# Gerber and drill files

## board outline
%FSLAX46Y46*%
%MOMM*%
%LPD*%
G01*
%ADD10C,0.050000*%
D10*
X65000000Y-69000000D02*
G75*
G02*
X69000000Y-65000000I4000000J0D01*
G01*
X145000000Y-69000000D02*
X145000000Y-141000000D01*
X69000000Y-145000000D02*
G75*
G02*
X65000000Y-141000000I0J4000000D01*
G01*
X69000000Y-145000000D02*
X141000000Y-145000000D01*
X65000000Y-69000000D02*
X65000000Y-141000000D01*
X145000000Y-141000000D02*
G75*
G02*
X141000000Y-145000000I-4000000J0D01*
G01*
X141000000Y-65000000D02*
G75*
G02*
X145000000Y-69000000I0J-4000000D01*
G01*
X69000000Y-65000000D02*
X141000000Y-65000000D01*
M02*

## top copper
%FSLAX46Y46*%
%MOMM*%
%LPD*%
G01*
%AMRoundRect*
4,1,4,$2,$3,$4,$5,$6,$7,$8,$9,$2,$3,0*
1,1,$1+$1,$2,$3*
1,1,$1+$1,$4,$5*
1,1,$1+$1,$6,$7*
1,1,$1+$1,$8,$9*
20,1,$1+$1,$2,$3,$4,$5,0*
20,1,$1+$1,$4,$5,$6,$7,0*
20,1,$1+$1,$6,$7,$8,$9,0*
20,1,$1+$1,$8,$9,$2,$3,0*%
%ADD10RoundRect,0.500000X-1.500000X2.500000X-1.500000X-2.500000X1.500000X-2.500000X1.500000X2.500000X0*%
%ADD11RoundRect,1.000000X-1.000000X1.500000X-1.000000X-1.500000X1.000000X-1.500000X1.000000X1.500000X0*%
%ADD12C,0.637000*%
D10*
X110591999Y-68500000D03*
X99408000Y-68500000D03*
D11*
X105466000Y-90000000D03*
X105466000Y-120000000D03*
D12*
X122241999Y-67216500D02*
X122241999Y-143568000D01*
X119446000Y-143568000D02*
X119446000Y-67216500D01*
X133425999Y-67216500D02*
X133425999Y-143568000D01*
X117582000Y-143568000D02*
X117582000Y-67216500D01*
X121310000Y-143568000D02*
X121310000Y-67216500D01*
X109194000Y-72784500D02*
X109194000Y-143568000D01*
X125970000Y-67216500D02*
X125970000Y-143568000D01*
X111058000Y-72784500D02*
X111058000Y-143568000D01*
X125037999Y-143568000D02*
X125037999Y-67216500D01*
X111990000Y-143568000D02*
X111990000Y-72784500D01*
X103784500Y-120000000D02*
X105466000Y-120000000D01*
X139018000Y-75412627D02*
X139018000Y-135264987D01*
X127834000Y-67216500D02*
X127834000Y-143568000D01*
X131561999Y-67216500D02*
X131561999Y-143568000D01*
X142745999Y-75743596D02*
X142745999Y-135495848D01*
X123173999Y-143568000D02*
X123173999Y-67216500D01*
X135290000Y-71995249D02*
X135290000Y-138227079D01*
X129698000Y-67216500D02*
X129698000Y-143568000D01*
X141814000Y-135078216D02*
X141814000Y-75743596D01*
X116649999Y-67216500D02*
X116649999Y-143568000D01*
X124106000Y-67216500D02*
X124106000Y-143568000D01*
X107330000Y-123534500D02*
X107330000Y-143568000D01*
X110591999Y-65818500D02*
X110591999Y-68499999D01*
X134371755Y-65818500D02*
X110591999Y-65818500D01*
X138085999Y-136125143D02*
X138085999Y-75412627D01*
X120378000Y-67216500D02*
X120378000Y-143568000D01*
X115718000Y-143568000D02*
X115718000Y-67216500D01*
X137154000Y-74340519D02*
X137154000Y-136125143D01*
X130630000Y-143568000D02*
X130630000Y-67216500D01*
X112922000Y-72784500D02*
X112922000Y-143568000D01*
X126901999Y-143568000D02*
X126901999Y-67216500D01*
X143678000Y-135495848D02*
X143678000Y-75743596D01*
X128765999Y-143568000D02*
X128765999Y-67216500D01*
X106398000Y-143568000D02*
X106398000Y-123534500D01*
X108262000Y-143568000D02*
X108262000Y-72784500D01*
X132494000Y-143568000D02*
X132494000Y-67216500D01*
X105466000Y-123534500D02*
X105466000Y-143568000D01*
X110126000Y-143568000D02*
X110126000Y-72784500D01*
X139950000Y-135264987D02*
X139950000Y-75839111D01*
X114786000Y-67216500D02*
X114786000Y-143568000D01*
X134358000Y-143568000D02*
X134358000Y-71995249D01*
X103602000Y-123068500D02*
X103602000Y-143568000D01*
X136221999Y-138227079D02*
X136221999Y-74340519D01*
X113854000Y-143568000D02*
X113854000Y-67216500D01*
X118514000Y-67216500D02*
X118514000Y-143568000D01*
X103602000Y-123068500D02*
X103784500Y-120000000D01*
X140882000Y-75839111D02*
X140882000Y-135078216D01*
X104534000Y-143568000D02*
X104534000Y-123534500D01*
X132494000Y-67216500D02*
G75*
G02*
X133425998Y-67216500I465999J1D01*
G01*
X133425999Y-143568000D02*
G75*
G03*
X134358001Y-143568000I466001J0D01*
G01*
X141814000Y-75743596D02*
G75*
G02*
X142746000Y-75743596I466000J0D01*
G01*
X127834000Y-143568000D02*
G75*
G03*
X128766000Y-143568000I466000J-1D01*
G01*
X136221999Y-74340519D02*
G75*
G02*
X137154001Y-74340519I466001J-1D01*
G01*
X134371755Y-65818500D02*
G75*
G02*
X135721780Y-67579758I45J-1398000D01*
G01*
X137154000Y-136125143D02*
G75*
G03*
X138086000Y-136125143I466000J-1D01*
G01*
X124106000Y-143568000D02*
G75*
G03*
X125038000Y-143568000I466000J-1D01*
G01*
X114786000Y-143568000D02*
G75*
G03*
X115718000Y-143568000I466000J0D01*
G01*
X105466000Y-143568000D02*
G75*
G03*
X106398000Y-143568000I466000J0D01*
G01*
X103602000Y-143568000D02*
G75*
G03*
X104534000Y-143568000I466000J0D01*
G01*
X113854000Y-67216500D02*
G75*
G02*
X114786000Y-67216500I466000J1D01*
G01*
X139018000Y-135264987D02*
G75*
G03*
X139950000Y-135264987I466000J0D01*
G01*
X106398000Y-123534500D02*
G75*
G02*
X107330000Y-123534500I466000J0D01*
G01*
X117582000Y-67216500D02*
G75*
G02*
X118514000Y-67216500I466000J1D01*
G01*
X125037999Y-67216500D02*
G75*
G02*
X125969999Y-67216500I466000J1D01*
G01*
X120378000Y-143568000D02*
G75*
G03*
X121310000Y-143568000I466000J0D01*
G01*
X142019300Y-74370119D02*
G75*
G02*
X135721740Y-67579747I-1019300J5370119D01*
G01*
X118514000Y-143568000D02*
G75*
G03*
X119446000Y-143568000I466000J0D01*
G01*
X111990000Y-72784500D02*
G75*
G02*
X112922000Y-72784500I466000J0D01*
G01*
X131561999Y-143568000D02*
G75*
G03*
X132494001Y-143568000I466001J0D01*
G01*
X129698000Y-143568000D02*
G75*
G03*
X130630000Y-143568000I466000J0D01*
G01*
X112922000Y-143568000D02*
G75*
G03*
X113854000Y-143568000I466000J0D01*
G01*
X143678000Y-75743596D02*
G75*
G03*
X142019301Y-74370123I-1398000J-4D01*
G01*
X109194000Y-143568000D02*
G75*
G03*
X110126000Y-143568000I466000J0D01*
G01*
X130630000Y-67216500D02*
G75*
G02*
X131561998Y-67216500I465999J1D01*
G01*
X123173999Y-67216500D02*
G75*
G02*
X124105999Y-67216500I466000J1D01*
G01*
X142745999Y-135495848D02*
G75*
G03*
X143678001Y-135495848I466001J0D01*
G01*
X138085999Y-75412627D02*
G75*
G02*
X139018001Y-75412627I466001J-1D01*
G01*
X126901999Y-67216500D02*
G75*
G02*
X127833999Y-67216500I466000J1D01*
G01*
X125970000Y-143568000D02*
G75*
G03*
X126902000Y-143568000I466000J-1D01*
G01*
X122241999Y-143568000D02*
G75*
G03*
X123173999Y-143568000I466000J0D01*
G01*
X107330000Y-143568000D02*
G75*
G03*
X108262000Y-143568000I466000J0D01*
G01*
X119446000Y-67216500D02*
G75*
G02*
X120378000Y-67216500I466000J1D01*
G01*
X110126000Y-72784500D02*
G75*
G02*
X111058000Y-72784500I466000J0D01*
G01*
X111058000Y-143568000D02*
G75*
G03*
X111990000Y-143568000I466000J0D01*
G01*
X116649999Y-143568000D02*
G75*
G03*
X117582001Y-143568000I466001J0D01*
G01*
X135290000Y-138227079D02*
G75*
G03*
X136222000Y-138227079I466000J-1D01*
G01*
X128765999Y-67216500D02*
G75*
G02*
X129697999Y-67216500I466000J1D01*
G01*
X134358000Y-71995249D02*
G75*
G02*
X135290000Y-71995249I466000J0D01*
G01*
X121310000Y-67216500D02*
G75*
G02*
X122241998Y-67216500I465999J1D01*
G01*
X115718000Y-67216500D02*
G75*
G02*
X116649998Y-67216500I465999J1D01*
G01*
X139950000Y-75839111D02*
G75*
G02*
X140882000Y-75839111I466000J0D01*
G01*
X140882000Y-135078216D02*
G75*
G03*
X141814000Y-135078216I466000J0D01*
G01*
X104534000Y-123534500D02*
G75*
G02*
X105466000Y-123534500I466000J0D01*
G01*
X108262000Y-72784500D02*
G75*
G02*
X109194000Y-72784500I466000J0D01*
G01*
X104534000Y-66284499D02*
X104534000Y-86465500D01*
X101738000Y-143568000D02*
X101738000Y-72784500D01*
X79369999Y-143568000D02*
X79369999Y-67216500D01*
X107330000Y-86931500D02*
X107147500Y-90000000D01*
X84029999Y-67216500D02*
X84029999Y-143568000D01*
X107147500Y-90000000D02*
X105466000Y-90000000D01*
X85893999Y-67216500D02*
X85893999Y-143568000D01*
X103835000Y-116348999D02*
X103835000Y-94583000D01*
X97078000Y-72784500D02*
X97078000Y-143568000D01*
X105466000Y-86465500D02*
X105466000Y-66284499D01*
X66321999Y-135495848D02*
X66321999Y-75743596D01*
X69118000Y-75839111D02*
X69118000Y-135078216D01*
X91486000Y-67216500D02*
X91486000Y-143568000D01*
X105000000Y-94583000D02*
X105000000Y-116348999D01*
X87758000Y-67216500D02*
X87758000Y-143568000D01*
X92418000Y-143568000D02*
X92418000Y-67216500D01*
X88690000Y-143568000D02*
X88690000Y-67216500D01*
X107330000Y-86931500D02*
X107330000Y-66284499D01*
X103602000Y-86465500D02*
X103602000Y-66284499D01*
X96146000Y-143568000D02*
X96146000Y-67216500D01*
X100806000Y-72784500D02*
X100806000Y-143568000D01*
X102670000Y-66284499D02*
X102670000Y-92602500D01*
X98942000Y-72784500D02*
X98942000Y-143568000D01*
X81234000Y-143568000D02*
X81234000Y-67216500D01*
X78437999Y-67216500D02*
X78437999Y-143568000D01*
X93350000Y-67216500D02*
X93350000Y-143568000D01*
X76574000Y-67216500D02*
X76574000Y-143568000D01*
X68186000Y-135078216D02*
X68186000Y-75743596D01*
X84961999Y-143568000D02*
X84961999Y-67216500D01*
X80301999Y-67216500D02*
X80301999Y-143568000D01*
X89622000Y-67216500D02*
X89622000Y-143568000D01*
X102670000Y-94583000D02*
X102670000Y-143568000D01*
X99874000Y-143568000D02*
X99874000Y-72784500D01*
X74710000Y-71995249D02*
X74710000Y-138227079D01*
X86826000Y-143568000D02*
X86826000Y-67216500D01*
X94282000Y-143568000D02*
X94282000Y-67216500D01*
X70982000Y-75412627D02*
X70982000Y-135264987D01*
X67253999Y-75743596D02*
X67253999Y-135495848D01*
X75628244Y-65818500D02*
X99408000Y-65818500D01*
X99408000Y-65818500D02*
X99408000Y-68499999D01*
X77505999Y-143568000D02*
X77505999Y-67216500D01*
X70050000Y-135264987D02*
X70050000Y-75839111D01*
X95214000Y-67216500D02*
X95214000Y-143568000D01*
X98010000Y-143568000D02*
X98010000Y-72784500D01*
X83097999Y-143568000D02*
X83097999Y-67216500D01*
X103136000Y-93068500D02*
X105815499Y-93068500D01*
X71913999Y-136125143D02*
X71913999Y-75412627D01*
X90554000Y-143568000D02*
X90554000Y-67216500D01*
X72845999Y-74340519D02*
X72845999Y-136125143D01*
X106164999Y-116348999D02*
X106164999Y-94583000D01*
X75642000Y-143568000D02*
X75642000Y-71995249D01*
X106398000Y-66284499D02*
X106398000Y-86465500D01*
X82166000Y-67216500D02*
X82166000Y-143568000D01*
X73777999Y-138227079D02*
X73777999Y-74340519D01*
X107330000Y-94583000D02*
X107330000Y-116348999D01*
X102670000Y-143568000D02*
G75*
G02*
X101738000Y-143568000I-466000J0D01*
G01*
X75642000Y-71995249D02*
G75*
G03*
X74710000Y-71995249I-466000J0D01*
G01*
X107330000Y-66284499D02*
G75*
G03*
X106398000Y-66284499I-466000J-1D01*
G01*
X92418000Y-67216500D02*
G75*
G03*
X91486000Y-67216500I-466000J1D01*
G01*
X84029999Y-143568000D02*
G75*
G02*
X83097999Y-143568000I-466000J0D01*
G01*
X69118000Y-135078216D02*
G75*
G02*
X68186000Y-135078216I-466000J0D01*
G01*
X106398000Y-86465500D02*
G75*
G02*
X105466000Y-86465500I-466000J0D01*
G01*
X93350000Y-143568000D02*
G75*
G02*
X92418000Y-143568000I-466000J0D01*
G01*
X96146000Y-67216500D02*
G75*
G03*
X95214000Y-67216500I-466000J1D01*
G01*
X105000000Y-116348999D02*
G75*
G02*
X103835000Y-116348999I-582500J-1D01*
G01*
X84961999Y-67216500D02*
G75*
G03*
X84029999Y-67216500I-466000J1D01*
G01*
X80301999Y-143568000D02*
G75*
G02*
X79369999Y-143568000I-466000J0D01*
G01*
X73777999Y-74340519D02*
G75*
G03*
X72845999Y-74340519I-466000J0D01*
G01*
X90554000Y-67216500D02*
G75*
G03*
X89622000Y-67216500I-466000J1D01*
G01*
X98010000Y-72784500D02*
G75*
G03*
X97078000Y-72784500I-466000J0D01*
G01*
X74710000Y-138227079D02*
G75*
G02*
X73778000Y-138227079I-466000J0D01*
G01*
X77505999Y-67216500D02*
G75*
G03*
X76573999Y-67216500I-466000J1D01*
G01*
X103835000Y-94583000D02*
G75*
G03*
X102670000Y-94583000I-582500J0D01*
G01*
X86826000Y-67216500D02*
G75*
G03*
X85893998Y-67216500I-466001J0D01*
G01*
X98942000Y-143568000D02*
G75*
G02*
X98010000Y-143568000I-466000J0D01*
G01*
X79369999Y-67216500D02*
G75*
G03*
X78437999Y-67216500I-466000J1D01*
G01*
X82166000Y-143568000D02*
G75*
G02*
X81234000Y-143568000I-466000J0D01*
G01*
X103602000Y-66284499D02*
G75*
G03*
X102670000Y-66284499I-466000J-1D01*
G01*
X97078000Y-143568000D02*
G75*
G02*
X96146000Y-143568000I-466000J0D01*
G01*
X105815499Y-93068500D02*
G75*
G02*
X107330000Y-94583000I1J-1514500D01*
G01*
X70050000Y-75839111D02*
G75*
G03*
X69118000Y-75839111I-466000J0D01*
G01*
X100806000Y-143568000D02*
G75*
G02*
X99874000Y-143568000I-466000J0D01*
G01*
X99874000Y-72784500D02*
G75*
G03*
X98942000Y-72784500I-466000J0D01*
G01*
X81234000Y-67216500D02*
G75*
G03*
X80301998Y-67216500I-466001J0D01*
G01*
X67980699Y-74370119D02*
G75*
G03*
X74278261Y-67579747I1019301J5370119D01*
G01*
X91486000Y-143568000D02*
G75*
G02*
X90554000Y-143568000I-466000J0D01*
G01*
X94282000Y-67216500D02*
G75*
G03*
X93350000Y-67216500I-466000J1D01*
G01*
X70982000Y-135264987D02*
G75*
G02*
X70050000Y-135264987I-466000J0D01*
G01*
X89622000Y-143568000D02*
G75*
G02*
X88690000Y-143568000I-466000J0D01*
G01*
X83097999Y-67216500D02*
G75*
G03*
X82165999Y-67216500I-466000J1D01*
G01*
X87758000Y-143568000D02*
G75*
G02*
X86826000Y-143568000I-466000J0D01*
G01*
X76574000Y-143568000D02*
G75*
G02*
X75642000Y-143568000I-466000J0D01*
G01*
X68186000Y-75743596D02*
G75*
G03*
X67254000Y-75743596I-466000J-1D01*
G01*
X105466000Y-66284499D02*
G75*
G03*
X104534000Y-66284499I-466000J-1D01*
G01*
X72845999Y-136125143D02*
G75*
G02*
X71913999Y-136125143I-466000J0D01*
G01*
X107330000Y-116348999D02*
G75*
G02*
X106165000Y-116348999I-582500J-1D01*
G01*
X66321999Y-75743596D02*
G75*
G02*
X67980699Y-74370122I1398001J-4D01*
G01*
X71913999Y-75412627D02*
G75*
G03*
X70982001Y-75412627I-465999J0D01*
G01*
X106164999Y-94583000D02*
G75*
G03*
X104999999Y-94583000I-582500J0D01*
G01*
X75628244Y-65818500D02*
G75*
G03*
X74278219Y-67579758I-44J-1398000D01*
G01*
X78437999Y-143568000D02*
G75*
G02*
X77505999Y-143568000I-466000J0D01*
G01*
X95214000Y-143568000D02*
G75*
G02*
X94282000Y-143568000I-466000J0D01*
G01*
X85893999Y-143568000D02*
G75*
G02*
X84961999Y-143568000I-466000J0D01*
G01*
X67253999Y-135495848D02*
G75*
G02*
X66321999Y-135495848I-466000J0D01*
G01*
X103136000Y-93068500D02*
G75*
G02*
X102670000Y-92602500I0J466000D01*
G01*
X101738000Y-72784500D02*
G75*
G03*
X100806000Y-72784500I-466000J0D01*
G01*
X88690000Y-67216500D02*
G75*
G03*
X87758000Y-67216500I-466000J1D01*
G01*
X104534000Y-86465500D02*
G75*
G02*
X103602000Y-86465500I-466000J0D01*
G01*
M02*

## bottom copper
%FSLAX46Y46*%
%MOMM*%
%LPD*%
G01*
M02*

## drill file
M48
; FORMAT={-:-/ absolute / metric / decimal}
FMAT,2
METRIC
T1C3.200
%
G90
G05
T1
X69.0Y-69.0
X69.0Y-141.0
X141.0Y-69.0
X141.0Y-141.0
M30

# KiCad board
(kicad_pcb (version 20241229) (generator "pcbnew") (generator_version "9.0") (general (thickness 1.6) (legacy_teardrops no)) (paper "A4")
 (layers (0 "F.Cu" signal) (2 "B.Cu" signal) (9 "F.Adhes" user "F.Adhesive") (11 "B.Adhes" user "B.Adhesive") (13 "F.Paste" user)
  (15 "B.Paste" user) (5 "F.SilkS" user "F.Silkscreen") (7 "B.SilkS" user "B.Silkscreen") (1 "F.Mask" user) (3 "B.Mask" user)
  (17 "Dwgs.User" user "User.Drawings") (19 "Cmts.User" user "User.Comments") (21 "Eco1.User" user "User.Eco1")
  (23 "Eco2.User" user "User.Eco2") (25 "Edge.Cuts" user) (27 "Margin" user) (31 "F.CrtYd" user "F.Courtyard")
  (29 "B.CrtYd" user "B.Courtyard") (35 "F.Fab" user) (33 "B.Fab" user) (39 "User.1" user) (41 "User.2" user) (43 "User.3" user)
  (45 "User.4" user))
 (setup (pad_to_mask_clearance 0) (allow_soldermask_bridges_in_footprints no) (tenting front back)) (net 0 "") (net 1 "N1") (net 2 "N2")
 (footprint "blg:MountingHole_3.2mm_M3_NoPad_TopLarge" (layer "F.Cu") (at 141 69)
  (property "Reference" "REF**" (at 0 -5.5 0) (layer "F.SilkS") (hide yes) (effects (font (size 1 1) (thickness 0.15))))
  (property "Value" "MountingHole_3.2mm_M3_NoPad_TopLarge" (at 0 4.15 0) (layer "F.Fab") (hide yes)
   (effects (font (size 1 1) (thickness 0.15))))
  (pad "" np_thru_hole circle (at 0 0) (size 7.6 7.6) (drill 3.2) (layers) (zone_connect 2)))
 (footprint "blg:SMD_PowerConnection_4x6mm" (layer "F.Cu") (at 110.591999 68.5 -90)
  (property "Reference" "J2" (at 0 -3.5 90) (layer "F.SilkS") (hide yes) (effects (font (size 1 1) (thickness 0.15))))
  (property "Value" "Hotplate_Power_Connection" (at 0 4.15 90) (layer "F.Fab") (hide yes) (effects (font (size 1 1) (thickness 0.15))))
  (pad "1" smd roundrect (at 0 0 270) (size 6 4) (layers "F.Cu" "F.Mask" "F.Paste") (roundrect_rratio 0.125) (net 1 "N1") (zone_connect 2)))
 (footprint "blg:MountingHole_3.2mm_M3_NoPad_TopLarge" (layer "F.Cu") (at 69 141)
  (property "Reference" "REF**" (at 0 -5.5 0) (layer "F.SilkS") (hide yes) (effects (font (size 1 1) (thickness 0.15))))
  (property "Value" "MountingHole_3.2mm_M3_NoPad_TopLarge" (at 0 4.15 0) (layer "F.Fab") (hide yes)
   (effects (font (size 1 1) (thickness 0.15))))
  (pad "" np_thru_hole circle (at 0 0) (size 7.6 7.6) (drill 3.2) (layers) (zone_connect 2)))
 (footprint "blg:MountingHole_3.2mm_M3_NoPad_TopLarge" (layer "F.Cu") (at 141 141)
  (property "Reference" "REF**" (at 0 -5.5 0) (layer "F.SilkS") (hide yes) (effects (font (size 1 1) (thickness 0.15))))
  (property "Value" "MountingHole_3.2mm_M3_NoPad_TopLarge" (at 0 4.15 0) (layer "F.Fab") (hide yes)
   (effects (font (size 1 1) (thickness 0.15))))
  (pad "" np_thru_hole circle (at 0 0) (size 7.6 7.6) (drill 3.2) (layers) (zone_connect 2)))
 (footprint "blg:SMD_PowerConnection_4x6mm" (layer "F.Cu") (at 99.408 68.5 -90)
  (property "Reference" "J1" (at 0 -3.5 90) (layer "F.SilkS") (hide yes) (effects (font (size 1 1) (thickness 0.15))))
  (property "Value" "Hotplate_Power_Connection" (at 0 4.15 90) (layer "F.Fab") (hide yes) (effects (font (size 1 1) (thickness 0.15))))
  (pad "1" smd roundrect (at 0 0 270) (size 6 4) (layers "F.Cu" "F.Mask" "F.Paste") (roundrect_rratio 0.125) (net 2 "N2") (zone_connect 2)))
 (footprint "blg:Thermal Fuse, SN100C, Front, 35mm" (layer "F.Cu") (at 105.466 105 -90)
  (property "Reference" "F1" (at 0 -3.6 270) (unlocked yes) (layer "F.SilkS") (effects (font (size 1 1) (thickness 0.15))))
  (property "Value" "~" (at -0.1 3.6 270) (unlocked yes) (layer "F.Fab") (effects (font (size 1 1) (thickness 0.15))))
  (pad "1" smd roundrect (at -15 0 270) (size 5 4) (layers "F.Cu" "F.Mask") (roundrect_rratio 0.25) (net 2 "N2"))
  (pad "2" smd roundrect (at 15 0 270) (size 5 4) (layers "F.Cu" "F.Mask") (roundrect_rratio 0.25) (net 1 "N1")))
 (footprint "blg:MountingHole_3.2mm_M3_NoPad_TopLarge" (layer "F.Cu") (at 69 69)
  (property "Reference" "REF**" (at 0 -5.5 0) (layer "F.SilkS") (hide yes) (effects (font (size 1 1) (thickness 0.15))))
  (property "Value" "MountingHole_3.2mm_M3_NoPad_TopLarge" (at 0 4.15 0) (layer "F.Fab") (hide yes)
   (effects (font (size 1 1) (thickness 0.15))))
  (pad "" np_thru_hole circle (at 0 0) (size 7.6 7.6) (drill 3.2) (layers) (zone_connect 2)))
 (gr_arc (start 65 69) (mid 66.171573 66.171573) (end 69 65) (stroke (width 0.05) (type solid)) (layer "Edge.Cuts"))
 (gr_line (start 145 69) (end 145 141) (stroke (width 0.05) (type default)) (layer "Edge.Cuts"))
 (gr_arc (start 69 145) (mid 66.171573 143.828427) (end 65 141) (stroke (width 0.05) (type solid)) (layer "Edge.Cuts"))
 (gr_line (start 69 145) (end 141 145) (stroke (width 0.05) (type default)) (layer "Edge.Cuts"))
 (gr_line (start 65 69) (end 65 141) (stroke (width 0.05) (type default)) (layer "Edge.Cuts"))
 (gr_arc (start 145 141) (mid 143.828427 143.828427) (end 141 145) (stroke (width 0.05) (type solid)) (layer "Edge.Cuts"))
 (gr_arc (start 141 65) (mid 143.828427 66.171573) (end 145 69) (stroke (width 0.05) (type solid)) (layer "Edge.Cuts"))
 (gr_line (start 69 65) (end 141 65) (stroke (width 0.05) (type default)) (layer "Edge.Cuts"))
 (segment (start 122.241999 67.2165) (end 122.241999 143.568) (width 0.637) (layer "F.Cu") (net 1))
 (segment (start 119.446 143.568) (end 119.446 67.2165) (width 0.637) (layer "F.Cu") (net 1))
 (segment (start 133.425999 67.2165) (end 133.425999 143.568) (width 0.637) (layer "F.Cu") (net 1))
 (segment (start 117.582 143.568) (end 117.582 67.2165) (width 0.637) (layer "F.Cu") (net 1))
 (segment (start 121.31 143.568) (end 121.31 67.2165) (width 0.637) (layer "F.Cu") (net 1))
 (segment (start 109.194 72.7845) (end 109.194 143.568) (width 0.637) (layer "F.Cu") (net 1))
 (segment (start 125.97 67.2165) (end 125.97 143.568) (width 0.637) (layer "F.Cu") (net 1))
 (segment (start 111.058 72.7845) (end 111.058 143.568) (width 0.637) (layer "F.Cu") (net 1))
 (segment (start 125.037999 143.568) (end 125.037999 67.2165) (width 0.637) (layer "F.Cu") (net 1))
 (segment (start 111.99 143.568) (end 111.99 72.7845) (width 0.637) (layer "F.Cu") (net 1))
 (segment (start 103.7845 120) (end 105.466 120) (width 0.637) (layer "F.Cu") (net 1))
 (segment (start 139.018 75.412627) (end 139.018 135.264987) (width 0.637) (layer "F.Cu") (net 1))
 (segment (start 127.834 67.2165) (end 127.834 143.568) (width 0.637) (layer "F.Cu") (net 1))
 (segment (start 131.561999 67.2165) (end 131.561999 143.568) (width 0.637) (layer "F.Cu") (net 1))
 (segment (start 142.745999 75.743596) (end 142.745999 135.495848) (width 0.637) (layer "F.Cu") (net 1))
 (segment (start 123.173999 143.568) (end 123.173999 67.2165) (width 0.637) (layer "F.Cu") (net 1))
 (segment (start 135.29 71.995249) (end 135.29 138.227079) (width 0.637) (layer "F.Cu") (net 1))
 (segment (start 129.698 67.2165) (end 129.698 143.568) (width 0.637) (layer "F.Cu") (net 1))
 (segment (start 141.814 135.078216) (end 141.814 75.743596) (width 0.637) (layer "F.Cu") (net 1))
 (segment (start 116.649999 67.2165) (end 116.649999 143.568) (width 0.637) (layer "F.Cu") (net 1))
 (segment (start 124.106 67.2165) (end 124.106 143.568) (width 0.637) (layer "F.Cu") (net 1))
 (segment (start 107.33 123.5345) (end 107.33 143.568) (width 0.637) (layer "F.Cu") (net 1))
 (segment (start 110.591999 65.8185) (end 110.591999 68.499999) (width 0.637) (layer "F.Cu") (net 1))
 (segment (start 134.371755 65.8185) (end 110.591999 65.8185) (width 0.637) (layer "F.Cu") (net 1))
 (segment (start 138.085999 136.125143) (end 138.085999 75.412627) (width 0.637) (layer "F.Cu") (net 1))
 (segment (start 120.378 67.2165) (end 120.378 143.568) (width 0.637) (layer "F.Cu") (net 1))
 (segment (start 115.718 143.568) (end 115.718 67.2165) (width 0.637) (layer "F.Cu") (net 1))
 (segment (start 137.154 74.340519) (end 137.154 136.125143) (width 0.637) (layer "F.Cu") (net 1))
 (segment (start 130.63 143.568) (end 130.63 67.2165) (width 0.637) (layer "F.Cu") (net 1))
 (segment (start 112.922 72.7845) (end 112.922 143.568) (width 0.637) (layer "F.Cu") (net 1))
 (segment (start 126.901999 143.568) (end 126.901999 67.2165) (width 0.637) (layer "F.Cu") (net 1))
 (segment (start 143.678 135.495848) (end 143.678 75.743596) (width 0.637) (layer "F.Cu") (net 1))
 (segment (start 128.765999 143.568) (end 128.765999 67.2165) (width 0.637) (layer "F.Cu") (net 1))
 (segment (start 106.398 143.568) (end 106.398 123.5345) (width 0.637) (layer "F.Cu") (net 1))
 (segment (start 108.262 143.568) (end 108.262 72.7845) (width 0.637) (layer "F.Cu") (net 1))
 (segment (start 132.494 143.568) (end 132.494 67.2165) (width 0.637) (layer "F.Cu") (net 1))
 (segment (start 105.466 123.5345) (end 105.466 143.568) (width 0.637) (layer "F.Cu") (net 1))
 (segment (start 110.126 143.568) (end 110.126 72.7845) (width 0.637) (layer "F.Cu") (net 1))
 (segment (start 139.95 135.264987) (end 139.95 75.839111) (width 0.637) (layer "F.Cu") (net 1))
 (segment (start 114.786 67.2165) (end 114.786 143.568) (width 0.637) (layer "F.Cu") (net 1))
 (segment (start 134.358 143.568) (end 134.358 71.995249) (width 0.637) (layer "F.Cu") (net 1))
 (segment (start 103.602 123.0685) (end 103.602 143.568) (width 0.637) (layer "F.Cu") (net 1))
 (segment (start 136.221999 138.227079) (end 136.221999 74.340519) (width 0.637) (layer "F.Cu") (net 1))
 (segment (start 113.854 143.568) (end 113.854 67.2165) (width 0.637) (layer "F.Cu") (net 1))
 (segment (start 118.514 67.2165) (end 118.514 143.568) (width 0.637) (layer "F.Cu") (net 1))
 (segment (start 103.602 123.0685) (end 103.7845 120) (width 0.637) (layer "F.Cu") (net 1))
 (segment (start 140.882 75.839111) (end 140.882 135.078216) (width 0.637) (layer "F.Cu") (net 1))
 (segment (start 104.534 143.568) (end 104.534 123.5345) (width 0.637) (layer "F.Cu") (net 1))
 (arc (start 132.494 67.2165) (mid 132.96 66.750499) (end 133.425999 67.2165) (width 0.637) (layer "F.Cu") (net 1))
 (arc (start 133.425999 143.568) (mid 133.892 144.034) (end 134.358 143.568) (width 0.637) (layer "F.Cu") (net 1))
 (arc (start 141.814 75.743596) (mid 142.28 75.277596) (end 142.745999 75.743596) (width 0.637) (layer "F.Cu") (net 1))
 (arc (start 127.834 143.568) (mid 128.3 144.034) (end 128.765999 143.568) (width 0.637) (layer "F.Cu") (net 1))
 (arc (start 136.221999 74.340519) (mid 136.688 73.874519) (end 137.154 74.340519) (width 0.637) (layer "F.Cu") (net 1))
 (arc (start 134.371755 65.8185) (mid 135.48131 66.366034) (end 135.721738 67.579747) (width 0.637) (layer "F.Cu") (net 1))
 (arc (start 137.154 136.125143) (mid 137.62 136.591143) (end 138.085999 136.125143) (width 0.637) (layer "F.Cu") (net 1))
 (arc (start 124.106 143.568) (mid 124.571999 144.034) (end 125.037999 143.568) (width 0.637) (layer "F.Cu") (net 1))
 (arc (start 114.786 143.568) (mid 115.252 144.034) (end 115.718 143.568) (width 0.637) (layer "F.Cu") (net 1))
 (arc (start 105.466 143.568) (mid 105.932 144.034) (end 106.398 143.568) (width 0.637) (layer "F.Cu") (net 1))
 (arc (start 103.602 143.568) (mid 104.068 144.034) (end 104.534 143.568) (width 0.637) (layer "F.Cu") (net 1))
 (arc (start 113.854 67.2165) (mid 114.32 66.750499) (end 114.786 67.2165) (width 0.637) (layer "F.Cu") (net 1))
 (arc (start 139.018 135.264987) (mid 139.484 135.730987) (end 139.95 135.264987) (width 0.637) (layer "F.Cu") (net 1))
 (arc (start 106.398 123.5345) (mid 106.864 123.0685) (end 107.33 123.5345) (width 0.637) (layer "F.Cu") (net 1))
 (arc (start 117.582 67.2165) (mid 118.048 66.750499) (end 118.514 67.2165) (width 0.637) (layer "F.Cu") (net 1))
 (arc (start 125.037999 67.2165) (mid 125.504 66.750499) (end 125.97 67.2165) (width 0.637) (layer "F.Cu") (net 1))
 (arc (start 120.378 143.568) (mid 120.844 144.034) (end 121.31 143.568) (width 0.637) (layer "F.Cu") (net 1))
 (arc (start 142.0193 74.370119) (mid 136.99226 72.716878) (end 135.721738 67.579747) (width 0.637) (layer "F.Cu") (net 1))
 (arc (start 118.514 143.568) (mid 118.979999 144.034) (end 119.446 143.568) (width 0.637) (layer "F.Cu") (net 1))
 (arc (start 111.99 72.7845) (mid 112.456 72.3185) (end 112.922 72.7845) (width 0.637) (layer "F.Cu") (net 1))
 (arc (start 131.561999 143.568) (mid 132.028 144.034) (end 132.494 143.568) (width 0.637) (layer "F.Cu") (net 1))
 (arc (start 129.698 143.568) (mid 130.164 144.034) (end 130.63 143.568) (width 0.637) (layer "F.Cu") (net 1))
 (arc (start 112.922 143.568) (mid 113.387999 144.034) (end 113.854 143.568) (width 0.637) (layer "F.Cu") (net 1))
 (arc (start 143.678 75.743596) (mid 143.322083 74.811681) (end 142.0193 74.370119) (width 0.637) (layer "F.Cu") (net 1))
 (arc (start 109.194 143.568) (mid 109.66 144.034) (end 110.126 143.568) (width 0.637) (layer "F.Cu") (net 1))
 (arc (start 130.63 67.2165) (mid 131.096 66.750499) (end 131.561999 67.2165) (width 0.637) (layer "F.Cu") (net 1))
 (arc (start 123.173999 67.2165) (mid 123.64 66.750499) (end 124.106 67.2165) (width 0.637) (layer "F.Cu") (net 1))
 (arc (start 142.745999 135.495848) (mid 143.212 135.961848) (end 143.678 135.495848) (width 0.637) (layer "F.Cu") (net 1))
 (arc (start 138.085999 75.412627) (mid 138.552 74.946627) (end 139.018 75.412627) (width 0.637) (layer "F.Cu") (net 1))
 (arc (start 126.901999 67.2165) (mid 127.367999 66.750499) (end 127.834 67.2165) (width 0.637) (layer "F.Cu") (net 1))
 (arc (start 125.97 143.568) (mid 126.436 144.034) (end 126.901999 143.568) (width 0.637) (layer "F.Cu") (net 1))
 (arc (start 122.241999 143.568) (mid 122.708 144.034) (end 123.173999 143.568) (width 0.637) (layer "F.Cu") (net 1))
 (arc (start 107.33 143.568) (mid 107.795999 144.034) (end 108.262 143.568) (width 0.637) (layer "F.Cu") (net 1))
 (arc (start 119.446 67.2165) (mid 119.911999 66.750499) (end 120.378 67.2165) (width 0.637) (layer "F.Cu") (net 1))
 (arc (start 110.126 72.7845) (mid 110.592 72.3185) (end 111.058 72.7845) (width 0.637) (layer "F.Cu") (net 1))
 (arc (start 111.058 143.568) (mid 111.524 144.034) (end 111.99 143.568) (width 0.637) (layer "F.Cu") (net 1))
 (arc (start 116.649999 143.568) (mid 117.116 144.034) (end 117.582 143.568) (width 0.637) (layer "F.Cu") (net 1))
 (arc (start 135.29 138.227079) (mid 135.756 138.693079) (end 136.221999 138.227079) (width 0.637) (layer "F.Cu") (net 1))
 (arc (start 128.765999 67.2165) (mid 129.232 66.750499) (end 129.698 67.2165) (width 0.637) (layer "F.Cu") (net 1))
 (arc (start 134.358 71.995249) (mid 134.824 71.529249) (end 135.29 71.995249) (width 0.637) (layer "F.Cu") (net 1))
 (arc (start 121.31 67.2165) (mid 121.776 66.750499) (end 122.241999 67.2165) (width 0.637) (layer "F.Cu") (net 1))
 (arc (start 115.718 67.2165) (mid 116.184 66.750499) (end 116.649999 67.2165) (width 0.637) (layer "F.Cu") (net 1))
 (arc (start 139.95 75.839111) (mid 140.416 75.373111) (end 140.882 75.839111) (width 0.637) (layer "F.Cu") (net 1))
 (arc (start 140.882 135.078216) (mid 141.348 135.544216) (end 141.814 135.078216) (width 0.637) (layer "F.Cu") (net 1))
 (arc (start 104.534 123.5345) (mid 105 123.0685) (end 105.466 123.5345) (width 0.637) (layer "F.Cu") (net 1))
 (arc (start 108.262 72.7845) (mid 108.728 72.3185) (end 109.194 72.7845) (width 0.637) (layer "F.Cu") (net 1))
 (segment (start 104.534 66.284499) (end 104.534 86.4655) (width 0.637) (layer "F.Cu") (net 2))
 (segment (start 101.738 143.568) (end 101.738 72.7845) (width 0.637) (layer "F.Cu") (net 2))
 (segment (start 79.369999 143.568) (end 79.369999 67.2165) (width 0.637) (layer "F.Cu") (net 2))
 (segment (start 107.33 86.9315) (end 107.1475 90) (width 0.637) (layer "F.Cu") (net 2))
 (segment (start 84.029999 67.2165) (end 84.029999 143.568) (width 0.637) (layer "F.Cu") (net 2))
 (segment (start 107.1475 90) (end 105.466 90) (width 0.637) (layer "F.Cu") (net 2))
 (segment (start 85.893999 67.2165) (end 85.893999 143.568) (width 0.637) (layer "F.Cu") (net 2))
 (segment (start 103.835 116.348999) (end 103.835 94.583) (width 0.637) (layer "F.Cu") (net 2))
 (segment (start 97.078 72.7845) (end 97.078 143.568) (width 0.637) (layer "F.Cu") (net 2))
 (segment (start 105.466 86.4655) (end 105.466 66.284499) (width 0.637) (layer "F.Cu") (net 2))
 (segment (start 66.321999 135.495848) (end 66.321999 75.743596) (width 0.637) (layer "F.Cu") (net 2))
 (segment (start 69.118 75.839111) (end 69.118 135.078216) (width 0.637) (layer "F.Cu") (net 2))
 (segment (start 91.486 67.2165) (end 91.486 143.568) (width 0.637) (layer "F.Cu") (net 2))
 (segment (start 105 94.583) (end 105 116.348999) (width 0.637) (layer "F.Cu") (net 2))
 (segment (start 87.758 67.2165) (end 87.758 143.568) (width 0.637) (layer "F.Cu") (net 2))
 (segment (start 92.418 143.568) (end 92.418 67.2165) (width 0.637) (layer "F.Cu") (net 2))
 (segment (start 88.69 143.568) (end 88.69 67.2165) (width 0.637) (layer "F.Cu") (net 2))
 (segment (start 107.33 86.9315) (end 107.33 66.284499) (width 0.637) (layer "F.Cu") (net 2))
 (segment (start 103.602 86.4655) (end 103.602 66.284499) (width 0.637) (layer "F.Cu") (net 2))
 (segment (start 96.146 143.568) (end 96.146 67.2165) (width 0.637) (layer "F.Cu") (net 2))
 (segment (start 100.806 72.7845) (end 100.806 143.568) (width 0.637) (layer "F.Cu") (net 2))
 (segment (start 102.67 66.284499) (end 102.67 92.6025) (width 0.637) (layer "F.Cu") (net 2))
 (segment (start 98.942 72.7845) (end 98.942 143.568) (width 0.637) (layer "F.Cu") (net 2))
 (segment (start 81.234 143.568) (end 81.234 67.2165) (width 0.637) (layer "F.Cu") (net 2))
 (segment (start 78.437999 67.2165) (end 78.437999 143.568) (width 0.637) (layer "F.Cu") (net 2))
 (segment (start 93.35 67.2165) (end 93.35 143.568) (width 0.637) (layer "F.Cu") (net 2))
 (segment (start 76.574 67.2165) (end 76.574 143.568) (width 0.637) (layer "F.Cu") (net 2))
 (segment (start 68.186 135.078216) (end 68.186 75.743596) (width 0.637) (layer "F.Cu") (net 2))
 (segment (start 84.961999 143.568) (end 84.961999 67.2165) (width 0.637) (layer "F.Cu") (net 2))
 (segment (start 80.301999 67.2165) (end 80.301999 143.568) (width 0.637) (layer "F.Cu") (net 2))
 (segment (start 89.622 67.2165) (end 89.622 143.568) (width 0.637) (layer "F.Cu") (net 2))
 (segment (start 102.67 94.583) (end 102.67 143.568) (width 0.637) (layer "F.Cu") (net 2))
 (segment (start 99.874 143.568) (end 99.874 72.7845) (width 0.637) (layer "F.Cu") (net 2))
 (segment (start 74.71 71.995249) (end 74.71 138.227079) (width 0.637) (layer "F.Cu") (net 2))
 (segment (start 86.826 143.568) (end 86.826 67.2165) (width 0.637) (layer "F.Cu") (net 2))
 (segment (start 94.282 143.568) (end 94.282 67.2165) (width 0.637) (layer "F.Cu") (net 2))
 (segment (start 70.982 75.412627) (end 70.982 135.264987) (width 0.637) (layer "F.Cu") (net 2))
 (segment (start 67.253999 75.743596) (end 67.253999 135.495848) (width 0.637) (layer "F.Cu") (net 2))
 (segment (start 75.628244 65.8185) (end 99.408 65.8185) (width 0.637) (layer "F.Cu") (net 2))
 (segment (start 99.408 65.8185) (end 99.408 68.499999) (width 0.637) (layer "F.Cu") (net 2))
 (segment (start 77.505999 143.568) (end 77.505999 67.2165) (width 0.637) (layer "F.Cu") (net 2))
 (segment (start 70.05 135.264987) (end 70.05 75.839111) (width 0.637) (layer "F.Cu") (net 2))
 (segment (start 95.214 67.2165) (end 95.214 143.568) (width 0.637) (layer "F.Cu") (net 2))
 (segment (start 98.01 143.568) (end 98.01 72.7845) (width 0.637) (layer "F.Cu") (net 2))
 (segment (start 83.097999 143.568) (end 83.097999 67.2165) (width 0.637) (layer "F.Cu") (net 2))
 (segment (start 103.136 93.0685) (end 105.815499 93.0685) (width 0.637) (layer "F.Cu") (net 2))
 (segment (start 71.913999 136.125143) (end 71.913999 75.412627) (width 0.637) (layer "F.Cu") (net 2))
 (segment (start 90.554 143.568) (end 90.554 67.2165) (width 0.637) (layer "F.Cu") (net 2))
 (segment (start 72.845999 74.340519) (end 72.845999 136.125143) (width 0.637) (layer "F.Cu") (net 2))
 (segment (start 106.164999 116.348999) (end 106.164999 94.583) (width 0.637) (layer "F.Cu") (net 2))
 (segment (start 75.642 143.568) (end 75.642 71.995249) (width 0.637) (layer "F.Cu") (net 2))
 (segment (start 106.398 66.284499) (end 106.398 86.4655) (width 0.637) (layer "F.Cu") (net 2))
 (segment (start 82.166 67.2165) (end 82.166 143.568) (width 0.637) (layer "F.Cu") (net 2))
 (segment (start 73.777999 138.227079) (end 73.777999 74.340519) (width 0.637) (layer "F.Cu") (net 2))
 (segment (start 107.33 94.583) (end 107.33 116.348999) (width 0.637) (layer "F.Cu") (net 2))
 (arc (start 102.67 143.568) (mid 102.204 144.034) (end 101.738 143.568) (width 0.637) (layer "F.Cu") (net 2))
 (arc (start 75.642 71.995249) (mid 75.175999 71.529249) (end 74.71 71.995249) (width 0.637) (layer "F.Cu") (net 2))
 (arc (start 107.33 66.284499) (mid 106.864 65.8185) (end 106.398 66.284499) (width 0.637) (layer "F.Cu") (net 2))
 (arc (start 92.418 67.2165) (mid 91.952 66.750499) (end 91.486 67.2165) (width 0.637) (layer "F.Cu") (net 2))
 (arc (start 84.029999 143.568) (mid 83.564 144.034) (end 83.097999 143.568) (width 0.637) (layer "F.Cu") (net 2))
 (arc (start 69.118 135.078216) (mid 68.651999 135.544216) (end 68.186 135.078216) (width 0.637) (layer "F.Cu") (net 2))
 (arc (start 106.398 86.4655) (mid 105.932 86.9315) (end 105.466 86.4655) (width 0.637) (layer "F.Cu") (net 2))
 (arc (start 93.35 143.568) (mid 92.884 144.034) (end 92.418 143.568) (width 0.637) (layer "F.Cu") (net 2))
 (arc (start 96.146 67.2165) (mid 95.68 66.750499) (end 95.214 67.2165) (width 0.637) (layer "F.Cu") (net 2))
 (arc (start 105 116.348999) (mid 104.417499 116.9315) (end 103.835 116.348999) (width 0.637) (layer "F.Cu") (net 2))
 (arc (start 84.961999 67.2165) (mid 84.496 66.750499) (end 84.029999 67.2165) (width 0.637) (layer "F.Cu") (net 2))
 (arc (start 80.301999 143.568) (mid 79.835999 144.034) (end 79.369999 143.568) (width 0.637) (layer "F.Cu") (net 2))
 (arc (start 73.777999 74.340519) (mid 73.312 73.874519) (end 72.845999 74.340519) (width 0.637) (layer "F.Cu") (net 2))
 (arc (start 90.554 67.2165) (mid 90.088 66.750499) (end 89.622 67.2165) (width 0.637) (layer "F.Cu") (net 2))
 (arc (start 98.01 72.7845) (mid 97.544 72.3185) (end 97.078 72.7845) (width 0.637) (layer "F.Cu") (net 2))
 (arc (start 74.71 138.227079) (mid 74.243999 138.693079) (end 73.777999 138.227079) (width 0.637) (layer "F.Cu") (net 2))
 (arc (start 77.505999 67.2165) (mid 77.039999 66.750499) (end 76.574 67.2165) (width 0.637) (layer "F.Cu") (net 2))
 (arc (start 103.835 94.583) (mid 103.2525 94.0005) (end 102.67 94.583) (width 0.637) (layer "F.Cu") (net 2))
 (arc (start 86.826 67.2165) (mid 86.359999 66.750499) (end 85.893999 67.2165) (width 0.637) (layer "F.Cu") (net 2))
 (arc (start 98.942 143.568) (mid 98.476 144.034) (end 98.01 143.568) (width 0.637) (layer "F.Cu") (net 2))
 (arc (start 79.369999 67.2165) (mid 78.904 66.750499) (end 78.437999 67.2165) (width 0.637) (layer "F.Cu") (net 2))
 (arc (start 82.166 143.568) (mid 81.699999 144.034) (end 81.234 143.568) (width 0.637) (layer "F.Cu") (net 2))
 (arc (start 103.602 66.284499) (mid 103.136 65.8185) (end 102.67 66.284499) (width 0.637) (layer "F.Cu") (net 2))
 (arc (start 97.078 143.568) (mid 96.612 144.034) (end 96.146 143.568) (width 0.637) (layer "F.Cu") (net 2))
 (arc (start 105.815499 93.0685) (mid 106.886413 93.512086) (end 107.33 94.583) (width 0.637) (layer "F.Cu") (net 2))
 (arc (start 70.05 75.839111) (mid 69.583999 75.373111) (end 69.118 75.839111) (width 0.637) (layer "F.Cu") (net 2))
 (arc (start 100.806 143.568) (mid 100.34 144.034) (end 99.874 143.568) (width 0.637) (layer "F.Cu") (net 2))
 (arc (start 99.874 72.7845) (mid 99.408 72.3185) (end 98.942 72.7845) (width 0.637) (layer "F.Cu") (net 2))
 (arc (start 81.234 67.2165) (mid 80.767999 66.750499) (end 80.301999 67.2165) (width 0.637) (layer "F.Cu") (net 2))
 (arc (start 67.980699 74.370119) (mid 73.007739 72.716878) (end 74.278261 67.579747) (width 0.637) (layer "F.Cu") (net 2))
 (arc (start 91.486 143.568) (mid 91.02 144.034) (end 90.554 143.568) (width 0.637) (layer "F.Cu") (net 2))
 (arc (start 94.282 67.2165) (mid 93.816 66.750499) (end 93.35 67.2165) (width 0.637) (layer "F.Cu") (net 2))
 (arc (start 70.982 135.264987) (mid 70.515999 135.730987) (end 70.05 135.264987) (width 0.637) (layer "F.Cu") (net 2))
 (arc (start 89.622 143.568) (mid 89.156 144.034) (end 88.69 143.568) (width 0.637) (layer "F.Cu") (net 2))
 (arc (start 83.097999 67.2165) (mid 82.631999 66.750499) (end 82.166 67.2165) (width 0.637) (layer "F.Cu") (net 2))
 (arc (start 87.758 143.568) (mid 87.292 144.034) (end 86.826 143.568) (width 0.637) (layer "F.Cu") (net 2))
 (arc (start 76.574 143.568) (mid 76.107999 144.034) (end 75.642 143.568) (width 0.637) (layer "F.Cu") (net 2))
 (arc (start 68.186 75.743596) (mid 67.72 75.277596) (end 67.253999 75.743596) (width 0.637) (layer "F.Cu") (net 2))
 (arc (start 105.466 66.284499) (mid 105 65.8185) (end 104.534 66.284499) (width 0.637) (layer "F.Cu") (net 2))
 (arc (start 72.845999 136.125143) (mid 72.38 136.591143) (end 71.913999 136.125143) (width 0.637) (layer "F.Cu") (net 2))
 (arc (start 107.33 116.348999) (mid 106.7475 116.9315) (end 106.164999 116.348999) (width 0.637) (layer "F.Cu") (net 2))
 (arc (start 66.321999 75.743596) (mid 66.677916 74.811681) (end 67.980699 74.370119) (width 0.637) (layer "F.Cu") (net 2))
 (arc (start 71.913999 75.412627) (mid 71.448 74.946627) (end 70.982 75.412627) (width 0.637) (layer "F.Cu") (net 2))
 (arc (start 106.164999 94.583) (mid 105.5825 94.0005) (end 105 94.583) (width 0.637) (layer "F.Cu") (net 2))
 (arc (start 75.628244 65.8185) (mid 74.518689 66.366034) (end 74.278261 67.579747) (width 0.637) (layer "F.Cu") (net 2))
 (arc (start 78.437999 143.568) (mid 77.972 144.034) (end 77.505999 143.568) (width 0.637) (layer "F.Cu") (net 2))
 (arc (start 95.214 143.568) (mid 94.748 144.034) (end 94.282 143.568) (width 0.637) (layer "F.Cu") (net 2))
 (arc (start 85.893999 143.568) (mid 85.427999 144.034) (end 84.961999 143.568) (width 0.637) (layer "F.Cu") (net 2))
 (arc (start 67.253999 135.495848) (mid 66.788 135.961848) (end 66.321999 135.495848) (width 0.637) (layer "F.Cu") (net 2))
 (arc (start 103.136 93.0685) (mid 102.806488 92.932011) (end 102.67 92.6025) (width 0.637) (layer "F.Cu") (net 2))
 (arc (start 101.738 72.7845) (mid 101.272 72.3185) (end 100.806 72.7845) (width 0.637) (layer "F.Cu") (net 2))
 (arc (start 88.69 67.2165) (mid 88.224 66.750499) (end 87.758 67.2165) (width 0.637) (layer "F.Cu") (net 2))
 (arc (start 104.534 86.4655) (mid 104.068 86.9315) (end 103.602 86.4655) (width 0.637) (layer "F.Cu") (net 2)))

